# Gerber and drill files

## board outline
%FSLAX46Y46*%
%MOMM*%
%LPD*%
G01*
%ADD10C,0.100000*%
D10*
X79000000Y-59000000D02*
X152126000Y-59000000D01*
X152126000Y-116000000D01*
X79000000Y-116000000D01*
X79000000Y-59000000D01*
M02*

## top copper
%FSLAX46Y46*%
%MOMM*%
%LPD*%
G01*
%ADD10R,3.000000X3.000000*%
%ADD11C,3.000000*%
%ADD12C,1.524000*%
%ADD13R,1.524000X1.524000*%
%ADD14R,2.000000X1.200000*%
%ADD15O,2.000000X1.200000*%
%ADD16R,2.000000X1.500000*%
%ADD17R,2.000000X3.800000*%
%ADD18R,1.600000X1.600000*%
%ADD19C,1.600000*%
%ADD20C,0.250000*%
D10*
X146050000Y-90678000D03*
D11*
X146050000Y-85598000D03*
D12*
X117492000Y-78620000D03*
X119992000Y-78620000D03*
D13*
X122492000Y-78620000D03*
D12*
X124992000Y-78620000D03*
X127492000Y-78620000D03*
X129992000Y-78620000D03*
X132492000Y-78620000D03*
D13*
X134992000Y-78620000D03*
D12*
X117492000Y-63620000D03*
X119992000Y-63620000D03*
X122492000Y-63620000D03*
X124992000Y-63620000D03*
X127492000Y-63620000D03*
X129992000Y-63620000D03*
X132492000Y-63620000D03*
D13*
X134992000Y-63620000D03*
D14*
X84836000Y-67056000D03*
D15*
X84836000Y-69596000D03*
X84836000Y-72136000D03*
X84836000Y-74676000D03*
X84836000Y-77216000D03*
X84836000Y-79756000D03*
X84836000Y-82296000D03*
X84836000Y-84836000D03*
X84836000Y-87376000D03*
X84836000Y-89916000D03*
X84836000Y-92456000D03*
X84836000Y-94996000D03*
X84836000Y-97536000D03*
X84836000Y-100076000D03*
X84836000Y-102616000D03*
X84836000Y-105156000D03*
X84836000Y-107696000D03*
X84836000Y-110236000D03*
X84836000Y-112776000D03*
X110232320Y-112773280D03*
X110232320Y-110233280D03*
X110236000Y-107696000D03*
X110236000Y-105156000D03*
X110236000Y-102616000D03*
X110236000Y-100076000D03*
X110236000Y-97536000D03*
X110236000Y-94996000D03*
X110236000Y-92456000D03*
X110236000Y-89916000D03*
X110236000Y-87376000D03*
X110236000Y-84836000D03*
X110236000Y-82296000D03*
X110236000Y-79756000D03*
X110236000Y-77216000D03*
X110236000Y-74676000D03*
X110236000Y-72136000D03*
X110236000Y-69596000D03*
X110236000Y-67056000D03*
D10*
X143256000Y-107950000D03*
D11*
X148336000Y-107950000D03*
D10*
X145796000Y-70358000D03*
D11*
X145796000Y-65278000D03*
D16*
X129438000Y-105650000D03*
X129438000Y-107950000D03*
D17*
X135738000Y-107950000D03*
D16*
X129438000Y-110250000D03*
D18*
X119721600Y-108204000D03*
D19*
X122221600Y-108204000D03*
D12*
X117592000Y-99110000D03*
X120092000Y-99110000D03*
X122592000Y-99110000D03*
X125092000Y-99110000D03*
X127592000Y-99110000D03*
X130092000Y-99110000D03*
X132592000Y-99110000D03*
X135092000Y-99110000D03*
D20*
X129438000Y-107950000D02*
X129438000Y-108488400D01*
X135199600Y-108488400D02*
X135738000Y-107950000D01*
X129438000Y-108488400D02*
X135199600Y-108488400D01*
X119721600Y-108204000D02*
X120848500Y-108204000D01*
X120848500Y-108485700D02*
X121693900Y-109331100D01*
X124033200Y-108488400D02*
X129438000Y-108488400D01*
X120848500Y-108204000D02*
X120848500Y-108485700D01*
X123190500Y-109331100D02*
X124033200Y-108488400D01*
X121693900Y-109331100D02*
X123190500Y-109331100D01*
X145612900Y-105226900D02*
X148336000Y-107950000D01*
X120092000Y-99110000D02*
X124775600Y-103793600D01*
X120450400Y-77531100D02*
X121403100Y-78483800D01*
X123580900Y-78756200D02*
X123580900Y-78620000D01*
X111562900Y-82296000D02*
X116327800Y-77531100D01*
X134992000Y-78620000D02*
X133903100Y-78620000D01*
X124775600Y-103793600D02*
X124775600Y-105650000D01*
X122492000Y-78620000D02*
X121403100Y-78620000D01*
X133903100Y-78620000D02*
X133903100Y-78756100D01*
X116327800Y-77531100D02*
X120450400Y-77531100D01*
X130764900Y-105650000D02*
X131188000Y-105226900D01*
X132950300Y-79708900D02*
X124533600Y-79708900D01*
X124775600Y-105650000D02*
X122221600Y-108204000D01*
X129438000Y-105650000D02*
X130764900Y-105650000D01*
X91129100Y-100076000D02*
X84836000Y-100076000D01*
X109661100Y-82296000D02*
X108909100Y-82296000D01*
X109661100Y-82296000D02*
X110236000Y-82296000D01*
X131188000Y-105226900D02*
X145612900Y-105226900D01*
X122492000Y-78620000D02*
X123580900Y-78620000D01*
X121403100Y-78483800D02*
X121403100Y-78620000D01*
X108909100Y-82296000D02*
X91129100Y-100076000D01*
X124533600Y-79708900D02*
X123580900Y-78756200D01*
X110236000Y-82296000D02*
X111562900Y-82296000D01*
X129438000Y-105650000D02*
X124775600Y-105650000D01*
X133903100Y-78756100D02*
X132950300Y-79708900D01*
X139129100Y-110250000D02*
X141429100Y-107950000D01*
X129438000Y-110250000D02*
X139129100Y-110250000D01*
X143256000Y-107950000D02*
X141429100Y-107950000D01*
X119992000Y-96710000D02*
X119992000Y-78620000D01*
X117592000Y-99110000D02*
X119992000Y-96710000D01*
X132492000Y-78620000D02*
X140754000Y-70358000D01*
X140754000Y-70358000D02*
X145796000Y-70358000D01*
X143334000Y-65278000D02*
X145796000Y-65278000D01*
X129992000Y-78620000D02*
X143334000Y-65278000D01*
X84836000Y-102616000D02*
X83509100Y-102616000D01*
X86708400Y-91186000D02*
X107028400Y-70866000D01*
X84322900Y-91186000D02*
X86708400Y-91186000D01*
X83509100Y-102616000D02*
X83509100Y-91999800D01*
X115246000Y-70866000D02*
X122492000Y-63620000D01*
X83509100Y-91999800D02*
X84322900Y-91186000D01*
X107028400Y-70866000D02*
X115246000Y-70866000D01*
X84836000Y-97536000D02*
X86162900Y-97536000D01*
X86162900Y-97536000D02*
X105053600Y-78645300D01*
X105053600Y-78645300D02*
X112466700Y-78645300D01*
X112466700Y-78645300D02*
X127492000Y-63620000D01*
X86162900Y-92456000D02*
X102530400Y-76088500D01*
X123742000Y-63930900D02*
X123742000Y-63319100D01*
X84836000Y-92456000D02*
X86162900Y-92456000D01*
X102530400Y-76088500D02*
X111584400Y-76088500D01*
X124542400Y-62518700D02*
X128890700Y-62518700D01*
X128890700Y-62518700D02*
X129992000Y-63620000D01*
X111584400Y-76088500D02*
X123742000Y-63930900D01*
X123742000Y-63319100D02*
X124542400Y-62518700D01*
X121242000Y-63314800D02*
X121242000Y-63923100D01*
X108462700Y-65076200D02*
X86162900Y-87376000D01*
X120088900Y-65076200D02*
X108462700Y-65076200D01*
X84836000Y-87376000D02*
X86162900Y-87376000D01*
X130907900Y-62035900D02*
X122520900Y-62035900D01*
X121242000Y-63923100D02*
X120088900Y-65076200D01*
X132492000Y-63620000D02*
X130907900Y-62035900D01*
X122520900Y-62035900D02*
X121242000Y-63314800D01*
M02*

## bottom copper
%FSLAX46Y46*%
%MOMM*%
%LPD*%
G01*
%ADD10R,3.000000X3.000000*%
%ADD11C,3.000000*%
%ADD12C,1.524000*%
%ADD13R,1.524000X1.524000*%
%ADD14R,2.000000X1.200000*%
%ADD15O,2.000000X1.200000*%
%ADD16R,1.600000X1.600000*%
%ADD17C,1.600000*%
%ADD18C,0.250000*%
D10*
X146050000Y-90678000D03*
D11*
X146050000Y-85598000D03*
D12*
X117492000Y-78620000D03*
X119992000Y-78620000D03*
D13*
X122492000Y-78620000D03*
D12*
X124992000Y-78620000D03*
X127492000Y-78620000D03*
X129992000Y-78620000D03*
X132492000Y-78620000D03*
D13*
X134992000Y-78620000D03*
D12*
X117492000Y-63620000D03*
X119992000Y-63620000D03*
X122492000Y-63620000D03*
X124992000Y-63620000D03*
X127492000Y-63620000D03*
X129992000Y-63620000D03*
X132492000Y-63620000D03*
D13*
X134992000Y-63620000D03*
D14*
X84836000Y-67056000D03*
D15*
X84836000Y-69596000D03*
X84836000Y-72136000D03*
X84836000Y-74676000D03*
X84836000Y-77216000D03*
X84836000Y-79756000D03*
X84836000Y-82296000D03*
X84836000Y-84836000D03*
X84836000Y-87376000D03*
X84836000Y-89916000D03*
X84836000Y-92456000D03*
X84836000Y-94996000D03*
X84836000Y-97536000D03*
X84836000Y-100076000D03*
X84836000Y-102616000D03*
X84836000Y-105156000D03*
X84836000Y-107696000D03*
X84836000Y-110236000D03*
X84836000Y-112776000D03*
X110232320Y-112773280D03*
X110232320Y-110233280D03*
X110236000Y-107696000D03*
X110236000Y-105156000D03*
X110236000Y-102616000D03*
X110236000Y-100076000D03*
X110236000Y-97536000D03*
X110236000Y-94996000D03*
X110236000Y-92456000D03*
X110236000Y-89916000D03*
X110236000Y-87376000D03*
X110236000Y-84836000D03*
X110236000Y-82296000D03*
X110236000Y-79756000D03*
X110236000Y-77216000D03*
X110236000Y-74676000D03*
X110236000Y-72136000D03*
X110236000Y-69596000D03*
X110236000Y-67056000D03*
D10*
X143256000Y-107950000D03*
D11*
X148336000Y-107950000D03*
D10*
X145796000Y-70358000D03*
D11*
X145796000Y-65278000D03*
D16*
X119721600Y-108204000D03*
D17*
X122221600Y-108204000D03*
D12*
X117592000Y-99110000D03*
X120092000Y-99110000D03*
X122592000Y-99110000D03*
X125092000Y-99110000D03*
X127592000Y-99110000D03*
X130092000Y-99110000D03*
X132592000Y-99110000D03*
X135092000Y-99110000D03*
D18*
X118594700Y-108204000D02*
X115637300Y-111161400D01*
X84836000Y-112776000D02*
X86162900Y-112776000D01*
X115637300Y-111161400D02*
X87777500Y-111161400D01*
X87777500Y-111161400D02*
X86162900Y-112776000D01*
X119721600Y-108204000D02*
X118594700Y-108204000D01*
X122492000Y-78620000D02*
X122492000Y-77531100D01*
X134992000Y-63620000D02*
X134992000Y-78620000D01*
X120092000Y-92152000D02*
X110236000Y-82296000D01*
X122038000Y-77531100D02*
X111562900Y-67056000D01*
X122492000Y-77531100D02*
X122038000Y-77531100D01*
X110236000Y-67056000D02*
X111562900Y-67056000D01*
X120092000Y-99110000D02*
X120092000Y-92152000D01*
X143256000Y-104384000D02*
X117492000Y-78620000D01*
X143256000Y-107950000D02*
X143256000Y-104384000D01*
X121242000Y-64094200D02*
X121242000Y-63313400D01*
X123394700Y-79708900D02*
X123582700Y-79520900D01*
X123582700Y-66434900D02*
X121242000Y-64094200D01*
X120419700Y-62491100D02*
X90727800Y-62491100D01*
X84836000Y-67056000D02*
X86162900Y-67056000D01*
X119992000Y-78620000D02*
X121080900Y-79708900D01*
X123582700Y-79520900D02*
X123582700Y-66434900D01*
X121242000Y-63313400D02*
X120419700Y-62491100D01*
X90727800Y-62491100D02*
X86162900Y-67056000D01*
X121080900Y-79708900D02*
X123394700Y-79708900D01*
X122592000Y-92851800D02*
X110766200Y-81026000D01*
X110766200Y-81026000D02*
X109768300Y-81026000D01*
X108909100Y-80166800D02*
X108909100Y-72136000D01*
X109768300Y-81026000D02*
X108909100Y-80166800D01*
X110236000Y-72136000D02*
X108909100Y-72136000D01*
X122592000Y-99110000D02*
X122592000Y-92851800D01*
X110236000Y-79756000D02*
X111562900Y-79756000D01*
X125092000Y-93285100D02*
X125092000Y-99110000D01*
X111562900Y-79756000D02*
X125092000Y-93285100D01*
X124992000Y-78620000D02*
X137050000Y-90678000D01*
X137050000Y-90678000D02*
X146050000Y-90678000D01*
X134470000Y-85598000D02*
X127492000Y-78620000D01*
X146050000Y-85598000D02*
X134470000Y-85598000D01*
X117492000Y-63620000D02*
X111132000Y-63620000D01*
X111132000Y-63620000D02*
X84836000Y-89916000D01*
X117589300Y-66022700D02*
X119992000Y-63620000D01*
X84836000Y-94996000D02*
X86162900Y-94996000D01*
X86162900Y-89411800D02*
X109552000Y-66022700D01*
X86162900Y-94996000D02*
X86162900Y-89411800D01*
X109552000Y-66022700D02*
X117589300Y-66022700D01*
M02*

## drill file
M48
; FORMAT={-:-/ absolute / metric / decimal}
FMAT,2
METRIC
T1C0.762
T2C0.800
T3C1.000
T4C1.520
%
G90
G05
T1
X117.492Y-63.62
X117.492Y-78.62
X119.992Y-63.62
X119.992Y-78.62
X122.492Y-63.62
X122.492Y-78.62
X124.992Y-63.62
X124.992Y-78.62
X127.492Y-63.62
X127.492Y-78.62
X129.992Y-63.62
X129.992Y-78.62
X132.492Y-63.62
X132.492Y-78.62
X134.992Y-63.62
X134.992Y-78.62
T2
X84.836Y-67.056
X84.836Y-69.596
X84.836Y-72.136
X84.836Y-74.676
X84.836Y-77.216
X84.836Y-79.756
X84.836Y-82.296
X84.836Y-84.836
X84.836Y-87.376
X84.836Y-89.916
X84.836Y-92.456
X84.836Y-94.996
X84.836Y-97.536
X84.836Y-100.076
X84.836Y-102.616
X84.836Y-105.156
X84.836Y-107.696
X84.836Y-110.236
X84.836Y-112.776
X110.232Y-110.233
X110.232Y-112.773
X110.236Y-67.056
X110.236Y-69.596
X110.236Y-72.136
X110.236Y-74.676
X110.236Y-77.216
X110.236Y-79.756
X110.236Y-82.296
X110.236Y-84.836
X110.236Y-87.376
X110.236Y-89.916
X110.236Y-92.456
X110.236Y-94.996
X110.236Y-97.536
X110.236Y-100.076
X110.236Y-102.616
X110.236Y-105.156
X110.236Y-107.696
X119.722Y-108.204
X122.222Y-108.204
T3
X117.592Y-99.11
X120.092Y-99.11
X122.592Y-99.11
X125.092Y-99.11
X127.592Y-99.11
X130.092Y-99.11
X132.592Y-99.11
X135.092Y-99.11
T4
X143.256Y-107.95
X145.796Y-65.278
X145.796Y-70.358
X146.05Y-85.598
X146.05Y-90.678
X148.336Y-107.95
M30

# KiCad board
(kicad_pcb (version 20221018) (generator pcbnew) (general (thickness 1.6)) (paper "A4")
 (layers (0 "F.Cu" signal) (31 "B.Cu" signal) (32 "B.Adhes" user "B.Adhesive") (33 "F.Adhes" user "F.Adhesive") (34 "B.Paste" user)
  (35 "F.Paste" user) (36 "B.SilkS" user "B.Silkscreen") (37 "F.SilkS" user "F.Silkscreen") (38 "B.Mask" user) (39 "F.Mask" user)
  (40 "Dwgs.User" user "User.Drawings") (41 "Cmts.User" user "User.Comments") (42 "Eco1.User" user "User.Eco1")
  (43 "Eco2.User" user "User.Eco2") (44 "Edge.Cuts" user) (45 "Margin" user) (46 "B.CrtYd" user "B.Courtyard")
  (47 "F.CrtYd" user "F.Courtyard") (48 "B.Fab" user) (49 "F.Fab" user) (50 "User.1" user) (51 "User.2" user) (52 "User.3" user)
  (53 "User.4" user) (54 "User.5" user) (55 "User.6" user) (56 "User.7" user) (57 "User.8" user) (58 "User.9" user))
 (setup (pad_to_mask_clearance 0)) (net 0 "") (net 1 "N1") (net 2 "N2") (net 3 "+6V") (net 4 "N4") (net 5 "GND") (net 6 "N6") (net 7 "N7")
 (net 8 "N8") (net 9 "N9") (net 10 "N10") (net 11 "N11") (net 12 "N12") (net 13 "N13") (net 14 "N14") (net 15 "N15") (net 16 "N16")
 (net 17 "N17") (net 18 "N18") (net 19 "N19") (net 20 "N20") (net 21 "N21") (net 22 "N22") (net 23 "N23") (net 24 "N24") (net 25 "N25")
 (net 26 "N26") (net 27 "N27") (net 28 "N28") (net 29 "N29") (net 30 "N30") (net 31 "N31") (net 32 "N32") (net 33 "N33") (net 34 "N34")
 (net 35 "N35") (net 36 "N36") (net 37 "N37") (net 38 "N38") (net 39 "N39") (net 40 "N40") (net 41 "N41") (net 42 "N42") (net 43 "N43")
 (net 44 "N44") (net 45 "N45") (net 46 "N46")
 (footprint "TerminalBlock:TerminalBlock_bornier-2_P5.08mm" (layer "F.Cu") (at 146.05 90.678 90)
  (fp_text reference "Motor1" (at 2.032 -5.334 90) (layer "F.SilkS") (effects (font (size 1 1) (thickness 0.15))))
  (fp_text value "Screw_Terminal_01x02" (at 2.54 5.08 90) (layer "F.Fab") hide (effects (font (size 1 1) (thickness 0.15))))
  (pad "1" thru_hole rect (at 0 0 90) (size 3 3) (drill 1.52) (layers "*.Cu" "*.Mask") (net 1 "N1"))
  (pad "2" thru_hole circle (at 5.08 0 90) (size 3 3) (drill 1.52) (layers "*.Cu" "*.Mask") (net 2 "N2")))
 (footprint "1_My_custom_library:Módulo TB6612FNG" (layer "F.Cu") (at 126.492 71.12 90)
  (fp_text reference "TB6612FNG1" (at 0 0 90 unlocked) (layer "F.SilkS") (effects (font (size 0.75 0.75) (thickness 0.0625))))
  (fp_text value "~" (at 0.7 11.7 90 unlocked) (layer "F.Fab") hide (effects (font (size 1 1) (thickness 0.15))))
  (pad "1" thru_hole circle (at -7.5 -9 90) (size 1.524 1.524) (drill 0.762) (layers "*.Cu" "*.Mask") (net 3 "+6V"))
  (pad "2" thru_hole circle (at -7.5 -6.5 90) (size 1.524 1.524) (drill 0.762) (layers "*.Cu" "*.Mask") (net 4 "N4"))
  (pad "3" thru_hole rect (at -7.5 -4 90) (size 1.524 1.524) (drill 0.762) (layers "*.Cu" "*.Mask") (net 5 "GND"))
  (pad "4" thru_hole circle (at -7.5 -1.5 90) (size 1.524 1.524) (drill 0.762) (layers "*.Cu" "*.Mask") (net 1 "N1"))
  (pad "5" thru_hole circle (at -7.5 1 90) (size 1.524 1.524) (drill 0.762) (layers "*.Cu" "*.Mask") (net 2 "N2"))
  (pad "6" thru_hole circle (at -7.5 3.5 90) (size 1.524 1.524) (drill 0.762) (layers "*.Cu" "*.Mask") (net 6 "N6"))
  (pad "7" thru_hole circle (at -7.5 6 90) (size 1.524 1.524) (drill 0.762) (layers "*.Cu" "*.Mask") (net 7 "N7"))
  (pad "8" thru_hole rect (at -7.5 8.5 90) (size 1.524 1.524) (drill 0.762) (layers "*.Cu" "*.Mask") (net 5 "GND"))
  (pad "9" thru_hole circle (at 7.5 -9 90) (size 1.524 1.524) (drill 0.762) (layers "*.Cu" "*.Mask") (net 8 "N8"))
  (pad "10" thru_hole circle (at 7.5 -6.5 90) (size 1.524 1.524) (drill 0.762) (layers "*.Cu" "*.Mask") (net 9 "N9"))
  (pad "11" thru_hole circle (at 7.5 -4 90) (size 1.524 1.524) (drill 0.762) (layers "*.Cu" "*.Mask") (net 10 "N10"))
  (pad "12" thru_hole circle (at 7.5 -1.5 90) (size 1.524 1.524) (drill 0.762) (layers "*.Cu" "*.Mask") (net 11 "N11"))
  (pad "13" thru_hole circle (at 7.5 1 90) (size 1.524 1.524) (drill 0.762) (layers "*.Cu" "*.Mask") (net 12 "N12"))
  (pad "14" thru_hole circle (at 7.5 3.5 90) (size 1.524 1.524) (drill 0.762) (layers "*.Cu" "*.Mask") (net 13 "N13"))
  (pad "15" thru_hole circle (at 7.5 6 90) (size 1.524 1.524) (drill 0.762) (layers "*.Cu" "*.Mask") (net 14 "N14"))
  (pad "16" thru_hole rect (at 7.5 8.5 90) (size 1.524 1.524) (drill 0.762) (layers "*.Cu" "*.Mask") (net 5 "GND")))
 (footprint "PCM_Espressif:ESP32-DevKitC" (layer "F.Cu") (at 84.836 67.056)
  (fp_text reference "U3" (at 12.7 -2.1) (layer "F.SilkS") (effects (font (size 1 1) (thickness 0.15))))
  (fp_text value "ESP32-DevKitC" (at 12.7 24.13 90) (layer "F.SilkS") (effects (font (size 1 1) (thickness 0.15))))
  (pad "1" thru_hole rect (at 0 0 270) (size 1.2 2) (drill 0.8) (layers "*.Cu" "*.Mask") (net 4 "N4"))
  (pad "2" thru_hole oval (at 0 2.54 270) (size 1.2 2) (drill 0.8) (layers "*.Cu" "*.Mask") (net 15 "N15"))
  (pad "3" thru_hole oval (at 0 5.08 270) (size 1.2 2) (drill 0.8) (layers "*.Cu" "*.Mask") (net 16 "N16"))
  (pad "4" thru_hole oval (at 0 7.62 270) (size 1.2 2) (drill 0.8) (layers "*.Cu" "*.Mask") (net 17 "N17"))
  (pad "5" thru_hole oval (at 0 10.16 270) (size 1.2 2) (drill 0.8) (layers "*.Cu" "*.Mask") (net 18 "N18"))
  (pad "6" thru_hole oval (at 0 12.7 270) (size 1.2 2) (drill 0.8) (layers "*.Cu" "*.Mask") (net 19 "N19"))
  (pad "7" thru_hole oval (at 0 15.24 270) (size 1.2 2) (drill 0.8) (layers "*.Cu" "*.Mask") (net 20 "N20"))
  (pad "8" thru_hole oval (at 0 17.78 270) (size 1.2 2) (drill 0.8) (layers "*.Cu" "*.Mask") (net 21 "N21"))
  (pad "9" thru_hole oval (at 0 20.32 270) (size 1.2 2) (drill 0.8) (layers "*.Cu" "*.Mask") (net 14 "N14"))
  (pad "10" thru_hole oval (at 0 22.86 270) (size 1.2 2) (drill 0.8) (layers "*.Cu" "*.Mask") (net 8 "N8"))
  (pad "11" thru_hole oval (at 0 25.4 270) (size 1.2 2) (drill 0.8) (layers "*.Cu" "*.Mask") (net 13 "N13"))
  (pad "12" thru_hole oval (at 0 27.94 270) (size 1.2 2) (drill 0.8) (layers "*.Cu" "*.Mask") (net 9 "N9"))
  (pad "13" thru_hole oval (at 0 30.48 270) (size 1.2 2) (drill 0.8) (layers "*.Cu" "*.Mask") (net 12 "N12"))
  (pad "14" thru_hole oval (at 0 33.02 270) (size 1.2 2) (drill 0.8) (layers "*.Cu" "*.Mask") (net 5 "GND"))
  (pad "15" thru_hole oval (at 0 35.56 270) (size 1.2 2) (drill 0.8) (layers "*.Cu" "*.Mask") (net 10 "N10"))
  (pad "16" thru_hole oval (at 0 38.1 270) (size 1.2 2) (drill 0.8) (layers "*.Cu" "*.Mask") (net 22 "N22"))
  (pad "17" thru_hole oval (at 0 40.64 270) (size 1.2 2) (drill 0.8) (layers "*.Cu" "*.Mask") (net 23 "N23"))
  (pad "18" thru_hole oval (at 0 43.18 270) (size 1.2 2) (drill 0.8) (layers "*.Cu" "*.Mask") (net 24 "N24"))
  (pad "19" thru_hole oval (at 0 45.72 270) (size 1.2 2) (drill 0.8) (layers "*.Cu" "*.Mask") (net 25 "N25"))
  (pad "20" thru_hole oval (at 25.39632 45.71728 270) (size 1.2 2) (drill 0.8) (layers "*.Cu" "*.Mask") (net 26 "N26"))
  (pad "21" thru_hole oval (at 25.39632 43.17728 270) (size 1.2 2) (drill 0.8) (layers "*.Cu" "*.Mask") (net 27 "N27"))
  (pad "22" thru_hole oval (at 25.4 40.64 270) (size 1.2 2) (drill 0.8) (layers "*.Cu" "*.Mask") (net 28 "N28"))
  (pad "23" thru_hole oval (at 25.4 38.1 270) (size 1.2 2) (drill 0.8) (layers "*.Cu" "*.Mask") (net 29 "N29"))
  (pad "24" thru_hole oval (at 25.4 35.56 270) (size 1.2 2) (drill 0.8) (layers "*.Cu" "*.Mask") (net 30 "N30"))
  (pad "25" thru_hole oval (at 25.4 33.02 270) (size 1.2 2) (drill 0.8) (layers "*.Cu" "*.Mask") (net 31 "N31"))
  (pad "26" thru_hole oval (at 25.4 30.48 270) (size 1.2 2) (drill 0.8) (layers "*.Cu" "*.Mask") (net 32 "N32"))
  (pad "27" thru_hole oval (at 25.4 27.94 270) (size 1.2 2) (drill 0.8) (layers "*.Cu" "*.Mask") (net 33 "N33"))
  (pad "28" thru_hole oval (at 25.4 25.4 270) (size 1.2 2) (drill 0.8) (layers "*.Cu" "*.Mask") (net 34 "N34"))
  (pad "29" thru_hole oval (at 25.4 22.86 270) (size 1.2 2) (drill 0.8) (layers "*.Cu" "*.Mask") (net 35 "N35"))
  (pad "30" thru_hole oval (at 25.4 20.32 270) (size 1.2 2) (drill 0.8) (layers "*.Cu" "*.Mask") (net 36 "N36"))
  (pad "31" thru_hole oval (at 25.4 17.78 270) (size 1.2 2) (drill 0.8) (layers "*.Cu" "*.Mask") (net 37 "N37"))
  (pad "32" thru_hole oval (at 25.4 15.24 270) (size 1.2 2) (drill 0.8) (layers "*.Cu" "*.Mask") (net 5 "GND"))
  (pad "33" thru_hole oval (at 25.4 12.7 270) (size 1.2 2) (drill 0.8) (layers "*.Cu" "*.Mask") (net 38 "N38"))
  (pad "34" thru_hole oval (at 25.4 10.16 270) (size 1.2 2) (drill 0.8) (layers "*.Cu" "*.Mask") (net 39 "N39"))
  (pad "35" thru_hole oval (at 25.4 7.62 270) (size 1.2 2) (drill 0.8) (layers "*.Cu" "*.Mask") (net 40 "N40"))
  (pad "36" thru_hole oval (at 25.4 5.08 270) (size 1.2 2) (drill 0.8) (layers "*.Cu" "*.Mask") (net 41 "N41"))
  (pad "37" thru_hole oval (at 25.4 2.54 270) (size 1.2 2) (drill 0.8) (layers "*.Cu" "*.Mask") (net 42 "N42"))
  (pad "38" thru_hole oval (at 25.4 0 270) (size 1.2 2) (drill 0.8) (layers "*.Cu" "*.Mask") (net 5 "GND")))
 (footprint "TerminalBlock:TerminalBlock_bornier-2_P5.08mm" (layer "F.Cu") (at 143.256 107.95)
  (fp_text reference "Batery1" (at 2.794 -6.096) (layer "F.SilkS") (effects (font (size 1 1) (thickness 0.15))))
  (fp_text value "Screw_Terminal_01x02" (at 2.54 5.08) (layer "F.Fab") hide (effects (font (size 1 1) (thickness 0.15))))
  (pad "1" thru_hole rect (at 0 0) (size 3 3) (drill 1.52) (layers "*.Cu" "*.Mask") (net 3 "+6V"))
  (pad "2" thru_hole circle (at 5.08 0) (size 3 3) (drill 1.52) (layers "*.Cu" "*.Mask") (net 5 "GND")))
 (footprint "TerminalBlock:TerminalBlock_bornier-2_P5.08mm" (layer "F.Cu") (at 145.796 70.358 90)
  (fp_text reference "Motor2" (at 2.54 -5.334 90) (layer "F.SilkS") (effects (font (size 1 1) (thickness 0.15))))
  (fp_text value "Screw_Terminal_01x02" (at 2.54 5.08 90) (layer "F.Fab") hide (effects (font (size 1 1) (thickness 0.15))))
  (pad "1" thru_hole rect (at 0 0 90) (size 3 3) (drill 1.52) (layers "*.Cu" "*.Mask") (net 7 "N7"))
  (pad "2" thru_hole circle (at 5.08 0 90) (size 3 3) (drill 1.52) (layers "*.Cu" "*.Mask") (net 6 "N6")))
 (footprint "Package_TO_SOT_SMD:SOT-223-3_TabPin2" (layer "F.Cu") (at 132.588 107.95)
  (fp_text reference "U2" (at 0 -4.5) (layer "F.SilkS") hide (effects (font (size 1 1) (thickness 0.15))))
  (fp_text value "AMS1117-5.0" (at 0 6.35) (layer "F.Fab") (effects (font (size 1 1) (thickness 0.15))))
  (pad "1" smd rect (at -3.15 -2.3) (size 2 1.5) (layers "F.Cu" "F.Paste" "F.Mask") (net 5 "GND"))
  (pad "2" smd rect (at -3.15 0) (size 2 1.5) (layers "F.Cu" "F.Paste" "F.Mask") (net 25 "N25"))
  (pad "2" smd rect (at 3.15 0) (size 2 3.8) (layers "F.Cu" "F.Paste" "F.Mask") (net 25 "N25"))
  (pad "3" smd rect (at -3.15 2.3) (size 2 1.5) (layers "F.Cu" "F.Paste" "F.Mask") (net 3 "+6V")))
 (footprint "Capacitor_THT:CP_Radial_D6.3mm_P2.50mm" (layer "F.Cu") (at 119.7216 108.204)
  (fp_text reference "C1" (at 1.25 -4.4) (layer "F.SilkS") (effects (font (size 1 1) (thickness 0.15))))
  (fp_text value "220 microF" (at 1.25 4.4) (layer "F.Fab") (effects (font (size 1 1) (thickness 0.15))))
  (pad "1" thru_hole rect (at 0 0) (size 1.6 1.6) (drill 0.8) (layers "*.Cu" "*.Mask") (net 25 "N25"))
  (pad "2" thru_hole circle (at 2.5 0) (size 1.6 1.6) (drill 0.8) (layers "*.Cu" "*.Mask") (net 5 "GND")))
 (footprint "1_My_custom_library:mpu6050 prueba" (layer "F.Cu") (at 116.592 100.11 90)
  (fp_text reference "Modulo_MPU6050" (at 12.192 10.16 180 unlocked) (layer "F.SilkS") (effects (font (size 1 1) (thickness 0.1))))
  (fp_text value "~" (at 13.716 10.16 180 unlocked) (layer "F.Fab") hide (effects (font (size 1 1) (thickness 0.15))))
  (pad "1" thru_hole circle (at 1 1 90) (size 1.524 1.524) (drill 1) (layers "*.Cu" "*.Mask") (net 4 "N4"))
  (pad "2" thru_hole circle (at 1 3.5 90) (size 1.524 1.524) (drill 1) (layers "*.Cu" "*.Mask") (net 5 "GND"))
  (pad "3" thru_hole circle (at 1 6 90) (size 1.524 1.524) (drill 1) (layers "*.Cu" "*.Mask") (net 41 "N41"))
  (pad "4" thru_hole circle (at 1 8.5 90) (size 1.524 1.524) (drill 1) (layers "*.Cu" "*.Mask") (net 38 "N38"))
  (pad "5" thru_hole circle (at 1 11 90) (size 1.524 1.524) (drill 1) (layers "*.Cu" "*.Mask") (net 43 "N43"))
  (pad "6" thru_hole circle (at 1 13.5 90) (size 1.524 1.524) (drill 1) (layers "*.Cu" "*.Mask") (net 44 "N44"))
  (pad "7" thru_hole circle (at 1 16 90) (size 1.524 1.524) (drill 1) (layers "*.Cu" "*.Mask") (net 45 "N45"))
  (pad "8" thru_hole circle (at 1 18.5 90) (size 1.524 1.524) (drill 1) (layers "*.Cu" "*.Mask") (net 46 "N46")))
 (gr_rect (start 79 59) (end 152.126 116) (stroke (width 0.1) (type solid)) (fill none) (layer "Edge.Cuts"))
 (segment (start 129.438 107.95) (end 129.438 108.4884) (width 0.25) (layer "F.Cu") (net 25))
 (segment (start 135.1996 108.4884) (end 135.738 107.95) (width 0.25) (layer "F.Cu") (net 25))
 (segment (start 129.438 108.4884) (end 135.1996 108.4884) (width 0.25) (layer "F.Cu") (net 25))
 (segment (start 119.7216 108.204) (end 120.8485 108.204) (width 0.25) (layer "F.Cu") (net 25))
 (segment (start 120.8485 108.4857) (end 121.6939 109.3311) (width 0.25) (layer "F.Cu") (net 25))
 (segment (start 124.0332 108.4884) (end 129.438 108.4884) (width 0.25) (layer "F.Cu") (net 25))
 (segment (start 120.8485 108.204) (end 120.8485 108.4857) (width 0.25) (layer "F.Cu") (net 25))
 (segment (start 123.1905 109.3311) (end 124.0332 108.4884) (width 0.25) (layer "F.Cu") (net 25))
 (segment (start 121.6939 109.3311) (end 123.1905 109.3311) (width 0.25) (layer "F.Cu") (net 25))
 (segment (start 118.5947 108.204) (end 115.6373 111.1614) (width 0.25) (layer "B.Cu") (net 25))
 (segment (start 84.836 112.776) (end 86.1629 112.776) (width 0.25) (layer "B.Cu") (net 25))
 (segment (start 115.6373 111.1614) (end 87.7775 111.1614) (width 0.25) (layer "B.Cu") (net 25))
 (segment (start 87.7775 111.1614) (end 86.1629 112.776) (width 0.25) (layer "B.Cu") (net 25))
 (segment (start 119.7216 108.204) (end 118.5947 108.204) (width 0.25) (layer "B.Cu") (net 25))
 (segment (start 145.6129 105.2269) (end 148.336 107.95) (width 0.25) (layer "F.Cu") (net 5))
 (segment (start 120.092 99.11) (end 124.7756 103.7936) (width 0.25) (layer "F.Cu") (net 5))
 (segment (start 120.4504 77.5311) (end 121.4031 78.4838) (width 0.25) (layer "F.Cu") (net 5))
 (segment (start 123.5809 78.7562) (end 123.5809 78.62) (width 0.25) (layer "F.Cu") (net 5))
 (segment (start 111.5629 82.296) (end 116.3278 77.5311) (width 0.25) (layer "F.Cu") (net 5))
 (segment (start 134.992 78.62) (end 133.9031 78.62) (width 0.25) (layer "F.Cu") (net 5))
 (segment (start 124.7756 103.7936) (end 124.7756 105.65) (width 0.25) (layer "F.Cu") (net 5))
 (segment (start 122.492 78.62) (end 121.4031 78.62) (width 0.25) (layer "F.Cu") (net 5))
 (segment (start 133.9031 78.62) (end 133.9031 78.7561) (width 0.25) (layer "F.Cu") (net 5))
 (segment (start 116.3278 77.5311) (end 120.4504 77.5311) (width 0.25) (layer "F.Cu") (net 5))
 (segment (start 130.7649 105.65) (end 131.188 105.2269) (width 0.25) (layer "F.Cu") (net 5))
 (segment (start 132.9503 79.7089) (end 124.5336 79.7089) (width 0.25) (layer "F.Cu") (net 5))
 (segment (start 124.7756 105.65) (end 122.2216 108.204) (width 0.25) (layer "F.Cu") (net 5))
 (segment (start 129.438 105.65) (end 130.7649 105.65) (width 0.25) (layer "F.Cu") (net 5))
 (segment (start 91.1291 100.076) (end 84.836 100.076) (width 0.25) (layer "F.Cu") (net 5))
 (segment (start 109.6611 82.296) (end 108.9091 82.296) (width 0.25) (layer "F.Cu") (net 5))
 (segment (start 109.6611 82.296) (end 110.236 82.296) (width 0.25) (layer "F.Cu") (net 5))
 (segment (start 131.188 105.2269) (end 145.6129 105.2269) (width 0.25) (layer "F.Cu") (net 5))
 (segment (start 122.492 78.62) (end 123.5809 78.62) (width 0.25) (layer "F.Cu") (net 5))
 (segment (start 121.4031 78.4838) (end 121.4031 78.62) (width 0.25) (layer "F.Cu") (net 5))
 (segment (start 108.9091 82.296) (end 91.1291 100.076) (width 0.25) (layer "F.Cu") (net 5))
 (segment (start 124.5336 79.7089) (end 123.5809 78.7562) (width 0.25) (layer "F.Cu") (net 5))
 (segment (start 110.236 82.296) (end 111.5629 82.296) (width 0.25) (layer "F.Cu") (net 5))
 (segment (start 129.438 105.65) (end 124.7756 105.65) (width 0.25) (layer "F.Cu") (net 5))
 (segment (start 133.9031 78.7561) (end 132.9503 79.7089) (width 0.25) (layer "F.Cu") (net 5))
 (segment (start 122.492 78.62) (end 122.492 77.5311) (width 0.25) (layer "B.Cu") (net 5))
 (segment (start 134.992 63.62) (end 134.992 78.62) (width 0.25) (layer "B.Cu") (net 5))
 (segment (start 120.092 92.152) (end 110.236 82.296) (width 0.25) (layer "B.Cu") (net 5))
 (segment (start 122.038 77.5311) (end 111.5629 67.056) (width 0.25) (layer "B.Cu") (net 5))
 (segment (start 122.492 77.5311) (end 122.038 77.5311) (width 0.25) (layer "B.Cu") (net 5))
 (segment (start 110.236 67.056) (end 111.5629 67.056) (width 0.25) (layer "B.Cu") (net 5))
 (segment (start 120.092 99.11) (end 120.092 92.152) (width 0.25) (layer "B.Cu") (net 5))
 (segment (start 139.1291 110.25) (end 141.4291 107.95) (width 0.25) (layer "F.Cu") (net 3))
 (segment (start 129.438 110.25) (end 139.1291 110.25) (width 0.25) (layer "F.Cu") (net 3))
 (segment (start 143.256 107.95) (end 141.4291 107.95) (width 0.25) (layer "F.Cu") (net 3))
 (segment (start 143.256 104.384) (end 117.492 78.62) (width 0.25) (layer "B.Cu") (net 3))
 (segment (start 143.256 107.95) (end 143.256 104.384) (width 0.25) (layer "B.Cu") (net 3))
 (segment (start 119.992 96.71) (end 119.992 78.62) (width 0.25) (layer "F.Cu") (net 4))
 (segment (start 117.592 99.11) (end 119.992 96.71) (width 0.25) (layer "F.Cu") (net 4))
 (segment (start 121.242 64.0942) (end 121.242 63.3134) (width 0.25) (layer "B.Cu") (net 4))
 (segment (start 123.3947 79.7089) (end 123.5827 79.5209) (width 0.25) (layer "B.Cu") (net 4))
 (segment (start 123.5827 66.4349) (end 121.242 64.0942) (width 0.25) (layer "B.Cu") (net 4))
 (segment (start 120.4197 62.4911) (end 90.7278 62.4911) (width 0.25) (layer "B.Cu") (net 4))
 (segment (start 84.836 67.056) (end 86.1629 67.056) (width 0.25) (layer "B.Cu") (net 4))
 (segment (start 119.992 78.62) (end 121.0809 79.7089) (width 0.25) (layer "B.Cu") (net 4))
 (segment (start 123.5827 79.5209) (end 123.5827 66.4349) (width 0.25) (layer "B.Cu") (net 4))
 (segment (start 121.242 63.3134) (end 120.4197 62.4911) (width 0.25) (layer "B.Cu") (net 4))
 (segment (start 90.7278 62.4911) (end 86.1629 67.056) (width 0.25) (layer "B.Cu") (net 4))
 (segment (start 121.0809 79.7089) (end 123.3947 79.7089) (width 0.25) (layer "B.Cu") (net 4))
 (segment (start 122.592 92.8518) (end 110.7662 81.026) (width 0.25) (layer "B.Cu") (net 41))
 (segment (start 110.7662 81.026) (end 109.7683 81.026) (width 0.25) (layer "B.Cu") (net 41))
 (segment (start 108.9091 80.1668) (end 108.9091 72.136) (width 0.25) (layer "B.Cu") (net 41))
 (segment (start 109.7683 81.026) (end 108.9091 80.1668) (width 0.25) (layer "B.Cu") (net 41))
 (segment (start 110.236 72.136) (end 108.9091 72.136) (width 0.25) (layer "B.Cu") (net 41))
 (segment (start 122.592 99.11) (end 122.592 92.8518) (width 0.25) (layer "B.Cu") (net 41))
 (segment (start 110.236 79.756) (end 111.5629 79.756) (width 0.25) (layer "B.Cu") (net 38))
 (segment (start 125.092 93.2851) (end 125.092 99.11) (width 0.25) (layer "B.Cu") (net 38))
 (segment (start 111.5629 79.756) (end 125.092 93.2851) (width 0.25) (layer "B.Cu") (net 38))
 (segment (start 124.992 78.62) (end 137.05 90.678) (width 0.25) (layer "B.Cu") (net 1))
 (segment (start 137.05 90.678) (end 146.05 90.678) (width 0.25) (layer "B.Cu") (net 1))
 (segment (start 134.47 85.598) (end 127.492 78.62) (width 0.25) (layer "B.Cu") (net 2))
 (segment (start 146.05 85.598) (end 134.47 85.598) (width 0.25) (layer "B.Cu") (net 2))
 (segment (start 132.492 78.62) (end 140.754 70.358) (width 0.25) (layer "F.Cu") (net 7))
 (segment (start 140.754 70.358) (end 145.796 70.358) (width 0.25) (layer "F.Cu") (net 7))
 (segment (start 143.334 65.278) (end 145.796 65.278) (width 0.25) (layer "F.Cu") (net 6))
 (segment (start 129.992 78.62) (end 143.334 65.278) (width 0.25) (layer "F.Cu") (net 6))
 (segment (start 117.492 63.62) (end 111.132 63.62) (width 0.25) (layer "B.Cu") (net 8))
 (segment (start 111.132 63.62) (end 84.836 89.916) (width 0.25) (layer "B.Cu") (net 8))
 (segment (start 117.5893 66.0227) (end 119.992 63.62) (width 0.25) (layer "B.Cu") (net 9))
 (segment (start 84.836 94.996) (end 86.1629 94.996) (width 0.25) (layer "B.Cu") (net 9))
 (segment (start 86.1629 89.4118) (end 109.552 66.0227) (width 0.25) (layer "B.Cu") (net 9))
 (segment (start 86.1629 94.996) (end 86.1629 89.4118) (width 0.25) (layer "B.Cu") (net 9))
 (segment (start 109.552 66.0227) (end 117.5893 66.0227) (width 0.25) (layer "B.Cu") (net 9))
 (segment (start 84.836 102.616) (end 83.5091 102.616) (width 0.25) (layer "F.Cu") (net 10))
 (segment (start 86.7084 91.186) (end 107.0284 70.866) (width 0.25) (layer "F.Cu") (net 10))
 (segment (start 84.3229 91.186) (end 86.7084 91.186) (width 0.25) (layer "F.Cu") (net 10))
 (segment (start 83.5091 102.616) (end 83.5091 91.9998) (width 0.25) (layer "F.Cu") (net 10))
 (segment (start 115.246 70.866) (end 122.492 63.62) (width 0.25) (layer "F.Cu") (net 10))
 (segment (start 83.5091 91.9998) (end 84.3229 91.186) (width 0.25) (layer "F.Cu") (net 10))
 (segment (start 107.0284 70.866) (end 115.246 70.866) (width 0.25) (layer "F.Cu") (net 10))
 (segment (start 84.836 97.536) (end 86.1629 97.536) (width 0.25) (layer "F.Cu") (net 12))
 (segment (start 86.1629 97.536) (end 105.0536 78.6453) (width 0.25) (layer "F.Cu") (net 12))
 (segment (start 105.0536 78.6453) (end 112.4667 78.6453) (width 0.25) (layer "F.Cu") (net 12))
 (segment (start 112.4667 78.6453) (end 127.492 63.62) (width 0.25) (layer "F.Cu") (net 12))
 (segment (start 86.1629 92.456) (end 102.5304 76.0885) (width 0.25) (layer "F.Cu") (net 13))
 (segment (start 123.742 63.9309) (end 123.742 63.3191) (width 0.25) (layer "F.Cu") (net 13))
 (segment (start 84.836 92.456) (end 86.1629 92.456) (width 0.25) (layer "F.Cu") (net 13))
 (segment (start 102.5304 76.0885) (end 111.5844 76.0885) (width 0.25) (layer "F.Cu") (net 13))
 (segment (start 124.5424 62.5187) (end 128.8907 62.5187) (width 0.25) (layer "F.Cu") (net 13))
 (segment (start 128.8907 62.5187) (end 129.992 63.62) (width 0.25) (layer "F.Cu") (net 13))
 (segment (start 111.5844 76.0885) (end 123.742 63.9309) (width 0.25) (layer "F.Cu") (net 13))
 (segment (start 123.742 63.3191) (end 124.5424 62.5187) (width 0.25) (layer "F.Cu") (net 13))
 (segment (start 121.242 63.3148) (end 121.242 63.9231) (width 0.25) (layer "F.Cu") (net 14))
 (segment (start 108.4627 65.0762) (end 86.1629 87.376) (width 0.25) (layer "F.Cu") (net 14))
 (segment (start 120.0889 65.0762) (end 108.4627 65.0762) (width 0.25) (layer "F.Cu") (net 14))
 (segment (start 84.836 87.376) (end 86.1629 87.376) (width 0.25) (layer "F.Cu") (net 14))
 (segment (start 130.9079 62.0359) (end 122.5209 62.0359) (width 0.25) (layer "F.Cu") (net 14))
 (segment (start 121.242 63.9231) (end 120.0889 65.0762) (width 0.25) (layer "F.Cu") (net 14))
 (segment (start 132.492 63.62) (end 130.9079 62.0359) (width 0.25) (layer "F.Cu") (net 14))
 (segment (start 122.5209 62.0359) (end 121.242 63.3148) (width 0.25) (layer "F.Cu") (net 14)))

